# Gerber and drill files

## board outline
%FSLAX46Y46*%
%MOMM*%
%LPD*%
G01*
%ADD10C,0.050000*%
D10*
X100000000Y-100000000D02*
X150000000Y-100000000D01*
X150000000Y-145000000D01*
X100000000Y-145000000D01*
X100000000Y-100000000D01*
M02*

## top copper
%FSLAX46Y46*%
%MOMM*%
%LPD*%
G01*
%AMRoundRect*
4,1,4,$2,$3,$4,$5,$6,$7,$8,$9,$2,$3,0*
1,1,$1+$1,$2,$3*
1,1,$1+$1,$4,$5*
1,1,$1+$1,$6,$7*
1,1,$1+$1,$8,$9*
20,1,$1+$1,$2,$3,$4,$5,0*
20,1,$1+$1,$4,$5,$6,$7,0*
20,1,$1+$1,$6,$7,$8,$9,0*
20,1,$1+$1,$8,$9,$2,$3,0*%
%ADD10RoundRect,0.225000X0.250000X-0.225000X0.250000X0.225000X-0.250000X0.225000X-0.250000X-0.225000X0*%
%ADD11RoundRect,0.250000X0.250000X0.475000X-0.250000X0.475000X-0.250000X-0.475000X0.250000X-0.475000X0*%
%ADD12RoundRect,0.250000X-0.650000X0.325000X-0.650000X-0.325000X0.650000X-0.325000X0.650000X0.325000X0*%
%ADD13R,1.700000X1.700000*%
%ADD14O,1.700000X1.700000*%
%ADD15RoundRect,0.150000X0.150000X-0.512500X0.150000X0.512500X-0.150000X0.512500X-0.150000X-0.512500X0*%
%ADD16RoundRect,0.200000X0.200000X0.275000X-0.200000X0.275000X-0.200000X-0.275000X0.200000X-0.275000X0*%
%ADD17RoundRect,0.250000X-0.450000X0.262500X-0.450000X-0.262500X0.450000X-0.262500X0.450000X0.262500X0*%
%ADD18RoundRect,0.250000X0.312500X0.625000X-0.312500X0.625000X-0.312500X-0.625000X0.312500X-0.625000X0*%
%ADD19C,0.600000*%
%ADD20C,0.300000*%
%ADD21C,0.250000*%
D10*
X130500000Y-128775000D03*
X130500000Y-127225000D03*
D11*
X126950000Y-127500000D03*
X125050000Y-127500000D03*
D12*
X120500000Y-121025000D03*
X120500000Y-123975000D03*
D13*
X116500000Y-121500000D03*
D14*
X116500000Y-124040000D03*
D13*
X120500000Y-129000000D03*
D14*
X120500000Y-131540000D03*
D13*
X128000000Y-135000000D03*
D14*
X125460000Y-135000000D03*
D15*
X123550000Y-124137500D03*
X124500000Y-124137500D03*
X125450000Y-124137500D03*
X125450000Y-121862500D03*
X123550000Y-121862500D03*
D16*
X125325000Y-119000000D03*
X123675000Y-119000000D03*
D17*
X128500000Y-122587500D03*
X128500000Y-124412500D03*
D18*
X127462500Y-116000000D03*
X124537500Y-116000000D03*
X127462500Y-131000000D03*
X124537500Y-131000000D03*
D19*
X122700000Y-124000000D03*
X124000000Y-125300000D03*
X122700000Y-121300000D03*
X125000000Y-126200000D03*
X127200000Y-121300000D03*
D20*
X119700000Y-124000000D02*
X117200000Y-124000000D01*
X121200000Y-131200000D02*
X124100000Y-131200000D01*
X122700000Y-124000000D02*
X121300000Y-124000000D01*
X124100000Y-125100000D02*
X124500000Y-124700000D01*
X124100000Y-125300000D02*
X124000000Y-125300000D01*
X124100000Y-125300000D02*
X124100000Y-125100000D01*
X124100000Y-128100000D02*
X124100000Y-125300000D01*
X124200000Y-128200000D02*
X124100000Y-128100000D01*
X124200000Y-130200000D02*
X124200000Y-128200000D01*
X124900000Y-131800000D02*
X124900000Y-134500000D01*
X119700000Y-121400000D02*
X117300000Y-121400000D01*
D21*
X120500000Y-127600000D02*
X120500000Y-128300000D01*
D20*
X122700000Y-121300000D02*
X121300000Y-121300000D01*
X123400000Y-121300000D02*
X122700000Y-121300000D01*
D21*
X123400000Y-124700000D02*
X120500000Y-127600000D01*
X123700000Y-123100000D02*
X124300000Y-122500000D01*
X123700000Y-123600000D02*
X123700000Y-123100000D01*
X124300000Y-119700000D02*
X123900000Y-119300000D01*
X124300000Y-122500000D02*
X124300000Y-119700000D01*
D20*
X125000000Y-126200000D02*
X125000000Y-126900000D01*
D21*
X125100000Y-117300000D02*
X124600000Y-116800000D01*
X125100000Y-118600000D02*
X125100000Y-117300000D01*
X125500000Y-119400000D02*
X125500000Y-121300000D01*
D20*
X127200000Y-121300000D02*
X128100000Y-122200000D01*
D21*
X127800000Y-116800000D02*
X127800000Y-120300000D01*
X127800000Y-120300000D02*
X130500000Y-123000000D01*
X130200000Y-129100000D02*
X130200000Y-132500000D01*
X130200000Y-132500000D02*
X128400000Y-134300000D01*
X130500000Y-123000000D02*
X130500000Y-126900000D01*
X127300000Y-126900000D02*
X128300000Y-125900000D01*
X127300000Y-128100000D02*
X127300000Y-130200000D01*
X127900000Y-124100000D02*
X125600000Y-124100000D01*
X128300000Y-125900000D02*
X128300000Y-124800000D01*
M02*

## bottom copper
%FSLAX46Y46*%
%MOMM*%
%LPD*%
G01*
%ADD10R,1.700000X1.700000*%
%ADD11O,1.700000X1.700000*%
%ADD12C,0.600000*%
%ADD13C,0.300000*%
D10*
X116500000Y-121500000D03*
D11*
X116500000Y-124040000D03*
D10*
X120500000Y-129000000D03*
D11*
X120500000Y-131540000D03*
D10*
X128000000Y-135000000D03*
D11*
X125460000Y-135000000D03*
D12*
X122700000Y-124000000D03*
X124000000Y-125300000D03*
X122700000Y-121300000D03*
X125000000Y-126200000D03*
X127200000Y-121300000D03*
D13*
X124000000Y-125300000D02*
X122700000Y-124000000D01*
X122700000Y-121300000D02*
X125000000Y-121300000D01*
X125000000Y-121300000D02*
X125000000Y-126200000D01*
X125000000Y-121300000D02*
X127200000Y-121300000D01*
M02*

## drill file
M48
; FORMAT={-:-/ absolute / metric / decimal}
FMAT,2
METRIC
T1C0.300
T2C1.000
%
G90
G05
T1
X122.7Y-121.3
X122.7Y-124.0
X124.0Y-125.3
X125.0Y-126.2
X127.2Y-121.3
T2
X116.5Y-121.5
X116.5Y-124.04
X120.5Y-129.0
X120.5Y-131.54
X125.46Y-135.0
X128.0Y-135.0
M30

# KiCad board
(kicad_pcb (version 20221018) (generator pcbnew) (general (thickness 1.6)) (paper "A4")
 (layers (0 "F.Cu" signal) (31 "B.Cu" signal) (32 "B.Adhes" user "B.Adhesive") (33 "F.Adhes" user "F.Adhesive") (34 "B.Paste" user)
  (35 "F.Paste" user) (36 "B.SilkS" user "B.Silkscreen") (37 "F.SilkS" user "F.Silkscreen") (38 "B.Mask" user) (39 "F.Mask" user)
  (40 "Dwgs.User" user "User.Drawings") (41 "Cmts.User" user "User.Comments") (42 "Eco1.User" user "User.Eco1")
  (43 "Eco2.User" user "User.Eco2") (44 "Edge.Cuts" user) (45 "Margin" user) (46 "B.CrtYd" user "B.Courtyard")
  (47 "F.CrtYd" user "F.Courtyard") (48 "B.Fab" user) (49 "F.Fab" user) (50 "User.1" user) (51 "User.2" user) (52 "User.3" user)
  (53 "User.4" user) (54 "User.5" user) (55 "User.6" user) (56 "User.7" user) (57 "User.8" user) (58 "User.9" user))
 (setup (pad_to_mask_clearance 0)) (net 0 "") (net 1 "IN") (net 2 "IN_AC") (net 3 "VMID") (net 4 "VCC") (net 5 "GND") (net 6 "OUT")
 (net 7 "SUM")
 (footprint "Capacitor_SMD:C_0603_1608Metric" (layer "F.Cu") (at 130.5 128 90)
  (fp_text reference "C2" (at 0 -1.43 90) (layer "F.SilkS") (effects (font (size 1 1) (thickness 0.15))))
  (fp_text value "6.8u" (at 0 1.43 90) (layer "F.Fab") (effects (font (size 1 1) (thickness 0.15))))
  (pad "1" smd roundrect (at -0.775 0 90) (size 0.9 0.95) (layers "F.Cu" "F.Paste" "F.Mask") (roundrect_rratio 0.25) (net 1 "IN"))
  (pad "2" smd roundrect (at 0.775 0 90) (size 0.9 0.95) (layers "F.Cu" "F.Paste" "F.Mask") (roundrect_rratio 0.25) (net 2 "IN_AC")))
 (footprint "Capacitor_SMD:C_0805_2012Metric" (layer "F.Cu") (at 126 127.5 180)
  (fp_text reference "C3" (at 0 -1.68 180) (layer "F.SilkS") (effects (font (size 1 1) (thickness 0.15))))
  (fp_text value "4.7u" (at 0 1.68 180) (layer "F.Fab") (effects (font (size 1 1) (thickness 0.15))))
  (pad "1" smd roundrect (at -0.95 0 180) (size 1 1.45) (layers "F.Cu" "F.Paste" "F.Mask") (roundrect_rratio 0.25) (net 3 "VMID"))
  (pad "2" smd roundrect (at 0.95 0 180) (size 1 1.45) (layers "F.Cu" "F.Paste" "F.Mask") (roundrect_rratio 0.25) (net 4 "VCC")))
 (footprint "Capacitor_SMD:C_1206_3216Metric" (layer "F.Cu") (at 120.5 122.5 -90)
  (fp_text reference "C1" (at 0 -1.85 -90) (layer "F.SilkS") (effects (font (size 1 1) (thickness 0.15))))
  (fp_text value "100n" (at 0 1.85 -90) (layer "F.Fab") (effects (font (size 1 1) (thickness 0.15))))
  (pad "1" smd roundrect (at -1.475 0 270) (size 1.15 1.8) (layers "F.Cu" "F.Paste" "F.Mask") (roundrect_rratio 0.217391) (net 4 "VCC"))
  (pad "2" smd roundrect (at 1.475 0 270) (size 1.15 1.8) (layers "F.Cu" "F.Paste" "F.Mask") (roundrect_rratio 0.217391) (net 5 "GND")))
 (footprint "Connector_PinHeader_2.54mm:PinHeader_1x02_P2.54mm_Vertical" (layer "F.Cu") (at 116.5 121.5)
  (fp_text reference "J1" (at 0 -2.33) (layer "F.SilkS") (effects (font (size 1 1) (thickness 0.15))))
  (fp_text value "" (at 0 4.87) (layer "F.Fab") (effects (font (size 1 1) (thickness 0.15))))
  (pad "1" thru_hole rect (at 0 0) (size 1.7 1.7) (drill 1) (layers "*.Cu" "*.Mask") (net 4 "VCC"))
  (pad "2" thru_hole oval (at 0 2.54) (size 1.7 1.7) (drill 1) (layers "*.Cu" "*.Mask") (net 5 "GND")))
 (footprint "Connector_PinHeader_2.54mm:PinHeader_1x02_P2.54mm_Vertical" (layer "F.Cu") (at 120.5 129)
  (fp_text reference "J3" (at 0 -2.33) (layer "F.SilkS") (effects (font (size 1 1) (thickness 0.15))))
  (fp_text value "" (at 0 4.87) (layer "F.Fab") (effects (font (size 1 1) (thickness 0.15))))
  (pad "1" thru_hole rect (at 0 0) (size 1.7 1.7) (drill 1) (layers "*.Cu" "*.Mask") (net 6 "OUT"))
  (pad "2" thru_hole oval (at 0 2.54) (size 1.7 1.7) (drill 1) (layers "*.Cu" "*.Mask") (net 5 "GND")))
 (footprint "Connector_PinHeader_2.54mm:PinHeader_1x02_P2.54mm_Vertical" (layer "F.Cu") (at 128 135 -90)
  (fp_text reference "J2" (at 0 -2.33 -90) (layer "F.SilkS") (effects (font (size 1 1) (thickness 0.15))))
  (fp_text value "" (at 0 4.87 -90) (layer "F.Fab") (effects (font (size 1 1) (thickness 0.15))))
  (pad "1" thru_hole rect (at 0 0 270) (size 1.7 1.7) (drill 1) (layers "*.Cu" "*.Mask") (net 1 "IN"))
  (pad "2" thru_hole oval (at 0 2.54 270) (size 1.7 1.7) (drill 1) (layers "*.Cu" "*.Mask") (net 5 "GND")))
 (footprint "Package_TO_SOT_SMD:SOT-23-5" (layer "F.Cu") (at 124.5 123 90)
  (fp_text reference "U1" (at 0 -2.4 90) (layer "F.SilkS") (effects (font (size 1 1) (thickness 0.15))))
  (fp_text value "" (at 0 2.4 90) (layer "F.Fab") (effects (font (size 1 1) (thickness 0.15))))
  (pad "1" smd roundrect (at -1.1375 -0.95 90) (size 1.325 0.6) (layers "F.Cu" "F.Paste" "F.Mask") (roundrect_rratio 0.25) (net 6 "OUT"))
  (pad "2" smd roundrect (at -1.1375 0 90) (size 1.325 0.6) (layers "F.Cu" "F.Paste" "F.Mask") (roundrect_rratio 0.25) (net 5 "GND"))
  (pad "3" smd roundrect (at -1.1375 0.95 90) (size 1.325 0.6) (layers "F.Cu" "F.Paste" "F.Mask") (roundrect_rratio 0.25) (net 3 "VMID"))
  (pad "4" smd roundrect (at 1.1375 0.95 90) (size 1.325 0.6) (layers "F.Cu" "F.Paste" "F.Mask") (roundrect_rratio 0.25) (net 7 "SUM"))
  (pad "5" smd roundrect (at 1.1375 -0.95 90) (size 1.325 0.6) (layers "F.Cu" "F.Paste" "F.Mask") (roundrect_rratio 0.25) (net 4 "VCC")))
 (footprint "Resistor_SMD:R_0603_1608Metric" (layer "F.Cu") (at 124.5 119 180)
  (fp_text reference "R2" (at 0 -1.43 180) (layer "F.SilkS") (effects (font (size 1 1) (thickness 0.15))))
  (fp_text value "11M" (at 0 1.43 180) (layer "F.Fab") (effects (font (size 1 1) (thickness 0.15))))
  (pad "1" smd roundrect (at -0.825 0 180) (size 0.8 0.95) (layers "F.Cu" "F.Paste" "F.Mask") (roundrect_rratio 0.25) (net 7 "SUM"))
  (pad "2" smd roundrect (at 0.825 0 180) (size 0.8 0.95) (layers "F.Cu" "F.Paste" "F.Mask") (roundrect_rratio 0.25) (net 6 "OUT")))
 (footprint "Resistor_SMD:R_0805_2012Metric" (layer "F.Cu") (at 128.5 123.5 -90)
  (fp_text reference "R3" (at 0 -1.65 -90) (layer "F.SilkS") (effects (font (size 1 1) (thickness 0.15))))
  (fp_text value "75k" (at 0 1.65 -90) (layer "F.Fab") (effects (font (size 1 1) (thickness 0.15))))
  (pad "1" smd roundrect (at -0.9125 0 270) (size 1.025 1.4) (layers "F.Cu" "F.Paste" "F.Mask") (roundrect_rratio 0.243902) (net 4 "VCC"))
  (pad "2" smd roundrect (at 0.9125 0 270) (size 1.025 1.4) (layers "F.Cu" "F.Paste" "F.Mask") (roundrect_rratio 0.243902) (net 3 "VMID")))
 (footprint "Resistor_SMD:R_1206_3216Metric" (layer "F.Cu") (at 126 116 180)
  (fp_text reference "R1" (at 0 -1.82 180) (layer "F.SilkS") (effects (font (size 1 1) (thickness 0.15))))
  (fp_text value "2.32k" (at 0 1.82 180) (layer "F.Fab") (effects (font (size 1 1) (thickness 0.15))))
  (pad "1" smd roundrect (at -1.4625 0 180) (size 1.125 1.75) (layers "F.Cu" "F.Paste" "F.Mask") (roundrect_rratio 0.222222) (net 2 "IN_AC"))
  (pad "2" smd roundrect (at 1.4625 0 180) (size 1.125 1.75) (layers "F.Cu" "F.Paste" "F.Mask") (roundrect_rratio 0.222222) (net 7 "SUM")))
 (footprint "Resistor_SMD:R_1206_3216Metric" (layer "F.Cu") (at 126 131 180)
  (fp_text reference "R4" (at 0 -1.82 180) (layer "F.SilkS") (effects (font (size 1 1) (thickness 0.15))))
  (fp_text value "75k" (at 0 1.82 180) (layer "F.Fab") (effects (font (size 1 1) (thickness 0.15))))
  (pad "1" smd roundrect (at -1.4625 0 180) (size 1.125 1.75) (layers "F.Cu" "F.Paste" "F.Mask") (roundrect_rratio 0.222222) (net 3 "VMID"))
  (pad "2" smd roundrect (at 1.4625 0 180) (size 1.125 1.75) (layers "F.Cu" "F.Paste" "F.Mask") (roundrect_rratio 0.222222) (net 5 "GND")))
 (gr_rect (start 100 100) (end 150 145) (stroke (width 0.05) (type default)) (fill none) (layer "Edge.Cuts"))
 (segment (start 119.7 124) (end 117.2 124) (width 0.3) (layer "F.Cu") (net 5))
 (segment (start 121.2 131.2) (end 124.1 131.2) (width 0.3) (layer "F.Cu") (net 5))
 (segment (start 122.7 124) (end 121.3 124) (width 0.3) (layer "F.Cu") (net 5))
 (segment (start 124.1 125.1) (end 124.5 124.7) (width 0.3) (layer "F.Cu") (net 5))
 (segment (start 124.1 125.3) (end 124 125.3) (width 0.3) (layer "F.Cu") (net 5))
 (segment (start 124.1 125.3) (end 124.1 125.1) (width 0.3) (layer "F.Cu") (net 5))
 (segment (start 124.1 128.1) (end 124.1 125.3) (width 0.3) (layer "F.Cu") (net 5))
 (segment (start 124.2 128.2) (end 124.1 128.1) (width 0.3) (layer "F.Cu") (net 5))
 (segment (start 124.2 130.2) (end 124.2 128.2) (width 0.3) (layer "F.Cu") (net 5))
 (segment (start 124.9 131.8) (end 124.9 134.5) (width 0.3) (layer "F.Cu") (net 5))
 (via (at 122.7 124) (size 0.6) (drill 0.3) (layers "F.Cu" "B.Cu") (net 5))
 (via (at 124 125.3) (size 0.6) (drill 0.3) (layers "F.Cu" "B.Cu") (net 5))
 (segment (start 119.7 121.4) (end 117.3 121.4) (width 0.3) (layer "F.Cu") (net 4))
 (segment (start 120.5 127.6) (end 120.5 128.3) (width 0.25) (layer "F.Cu") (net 6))
 (segment (start 122.7 121.3) (end 121.3 121.3) (width 0.3) (layer "F.Cu") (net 4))
 (segment (start 123.4 121.3) (end 122.7 121.3) (width 0.3) (layer "F.Cu") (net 4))
 (segment (start 123.4 124.7) (end 120.5 127.6) (width 0.25) (layer "F.Cu") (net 6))
 (segment (start 123.7 123.1) (end 124.3 122.5) (width 0.25) (layer "F.Cu") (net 6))
 (segment (start 123.7 123.6) (end 123.7 123.1) (width 0.25) (layer "F.Cu") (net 6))
 (segment (start 124 125.3) (end 122.7 124) (width 0.3) (layer "B.Cu") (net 5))
 (segment (start 124.3 119.7) (end 123.9 119.3) (width 0.25) (layer "F.Cu") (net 6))
 (segment (start 124.3 122.5) (end 124.3 119.7) (width 0.25) (layer "F.Cu") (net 6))
 (segment (start 125 126.2) (end 125 126.9) (width 0.3) (layer "F.Cu") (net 4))
 (segment (start 125.1 117.3) (end 124.6 116.8) (width 0.25) (layer "F.Cu") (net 7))
 (segment (start 125.1 118.6) (end 125.1 117.3) (width 0.25) (layer "F.Cu") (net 7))
 (segment (start 125.5 119.4) (end 125.5 121.3) (width 0.25) (layer "F.Cu") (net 7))
 (segment (start 127.2 121.3) (end 128.1 122.2) (width 0.3) (layer "F.Cu") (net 4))
 (segment (start 127.8 116.8) (end 127.8 120.3) (width 0.25) (layer "F.Cu") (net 2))
 (segment (start 127.8 120.3) (end 130.5 123) (width 0.25) (layer "F.Cu") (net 2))
 (segment (start 130.2 129.1) (end 130.2 132.5) (width 0.25) (layer "F.Cu") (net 1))
 (segment (start 130.2 132.5) (end 128.4 134.3) (width 0.25) (layer "F.Cu") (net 1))
 (segment (start 130.5 123) (end 130.5 126.9) (width 0.25) (layer "F.Cu") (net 2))
 (via (at 122.7 121.3) (size 0.6) (drill 0.3) (layers "F.Cu" "B.Cu") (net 4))
 (via (at 125 126.2) (size 0.6) (drill 0.3) (layers "F.Cu" "B.Cu") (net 4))
 (via (at 127.2 121.3) (size 0.6) (drill 0.3) (layers "F.Cu" "B.Cu") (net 4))
 (segment (start 122.7 121.3) (end 125 121.3) (width 0.3) (layer "B.Cu") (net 4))
 (segment (start 125 121.3) (end 125 126.2) (width 0.3) (layer "B.Cu") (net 4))
 (segment (start 125 121.3) (end 127.2 121.3) (width 0.3) (layer "B.Cu") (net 4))
 (segment (start 127.3 126.9) (end 128.3 125.9) (width 0.25) (layer "F.Cu") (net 3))
 (segment (start 127.3 128.1) (end 127.3 130.2) (width 0.25) (layer "F.Cu") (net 3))
 (segment (start 127.9 124.1) (end 125.6 124.1) (width 0.25) (layer "F.Cu") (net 3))
 (segment (start 128.3 125.9) (end 128.3 124.8) (width 0.25) (layer "F.Cu") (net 3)))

